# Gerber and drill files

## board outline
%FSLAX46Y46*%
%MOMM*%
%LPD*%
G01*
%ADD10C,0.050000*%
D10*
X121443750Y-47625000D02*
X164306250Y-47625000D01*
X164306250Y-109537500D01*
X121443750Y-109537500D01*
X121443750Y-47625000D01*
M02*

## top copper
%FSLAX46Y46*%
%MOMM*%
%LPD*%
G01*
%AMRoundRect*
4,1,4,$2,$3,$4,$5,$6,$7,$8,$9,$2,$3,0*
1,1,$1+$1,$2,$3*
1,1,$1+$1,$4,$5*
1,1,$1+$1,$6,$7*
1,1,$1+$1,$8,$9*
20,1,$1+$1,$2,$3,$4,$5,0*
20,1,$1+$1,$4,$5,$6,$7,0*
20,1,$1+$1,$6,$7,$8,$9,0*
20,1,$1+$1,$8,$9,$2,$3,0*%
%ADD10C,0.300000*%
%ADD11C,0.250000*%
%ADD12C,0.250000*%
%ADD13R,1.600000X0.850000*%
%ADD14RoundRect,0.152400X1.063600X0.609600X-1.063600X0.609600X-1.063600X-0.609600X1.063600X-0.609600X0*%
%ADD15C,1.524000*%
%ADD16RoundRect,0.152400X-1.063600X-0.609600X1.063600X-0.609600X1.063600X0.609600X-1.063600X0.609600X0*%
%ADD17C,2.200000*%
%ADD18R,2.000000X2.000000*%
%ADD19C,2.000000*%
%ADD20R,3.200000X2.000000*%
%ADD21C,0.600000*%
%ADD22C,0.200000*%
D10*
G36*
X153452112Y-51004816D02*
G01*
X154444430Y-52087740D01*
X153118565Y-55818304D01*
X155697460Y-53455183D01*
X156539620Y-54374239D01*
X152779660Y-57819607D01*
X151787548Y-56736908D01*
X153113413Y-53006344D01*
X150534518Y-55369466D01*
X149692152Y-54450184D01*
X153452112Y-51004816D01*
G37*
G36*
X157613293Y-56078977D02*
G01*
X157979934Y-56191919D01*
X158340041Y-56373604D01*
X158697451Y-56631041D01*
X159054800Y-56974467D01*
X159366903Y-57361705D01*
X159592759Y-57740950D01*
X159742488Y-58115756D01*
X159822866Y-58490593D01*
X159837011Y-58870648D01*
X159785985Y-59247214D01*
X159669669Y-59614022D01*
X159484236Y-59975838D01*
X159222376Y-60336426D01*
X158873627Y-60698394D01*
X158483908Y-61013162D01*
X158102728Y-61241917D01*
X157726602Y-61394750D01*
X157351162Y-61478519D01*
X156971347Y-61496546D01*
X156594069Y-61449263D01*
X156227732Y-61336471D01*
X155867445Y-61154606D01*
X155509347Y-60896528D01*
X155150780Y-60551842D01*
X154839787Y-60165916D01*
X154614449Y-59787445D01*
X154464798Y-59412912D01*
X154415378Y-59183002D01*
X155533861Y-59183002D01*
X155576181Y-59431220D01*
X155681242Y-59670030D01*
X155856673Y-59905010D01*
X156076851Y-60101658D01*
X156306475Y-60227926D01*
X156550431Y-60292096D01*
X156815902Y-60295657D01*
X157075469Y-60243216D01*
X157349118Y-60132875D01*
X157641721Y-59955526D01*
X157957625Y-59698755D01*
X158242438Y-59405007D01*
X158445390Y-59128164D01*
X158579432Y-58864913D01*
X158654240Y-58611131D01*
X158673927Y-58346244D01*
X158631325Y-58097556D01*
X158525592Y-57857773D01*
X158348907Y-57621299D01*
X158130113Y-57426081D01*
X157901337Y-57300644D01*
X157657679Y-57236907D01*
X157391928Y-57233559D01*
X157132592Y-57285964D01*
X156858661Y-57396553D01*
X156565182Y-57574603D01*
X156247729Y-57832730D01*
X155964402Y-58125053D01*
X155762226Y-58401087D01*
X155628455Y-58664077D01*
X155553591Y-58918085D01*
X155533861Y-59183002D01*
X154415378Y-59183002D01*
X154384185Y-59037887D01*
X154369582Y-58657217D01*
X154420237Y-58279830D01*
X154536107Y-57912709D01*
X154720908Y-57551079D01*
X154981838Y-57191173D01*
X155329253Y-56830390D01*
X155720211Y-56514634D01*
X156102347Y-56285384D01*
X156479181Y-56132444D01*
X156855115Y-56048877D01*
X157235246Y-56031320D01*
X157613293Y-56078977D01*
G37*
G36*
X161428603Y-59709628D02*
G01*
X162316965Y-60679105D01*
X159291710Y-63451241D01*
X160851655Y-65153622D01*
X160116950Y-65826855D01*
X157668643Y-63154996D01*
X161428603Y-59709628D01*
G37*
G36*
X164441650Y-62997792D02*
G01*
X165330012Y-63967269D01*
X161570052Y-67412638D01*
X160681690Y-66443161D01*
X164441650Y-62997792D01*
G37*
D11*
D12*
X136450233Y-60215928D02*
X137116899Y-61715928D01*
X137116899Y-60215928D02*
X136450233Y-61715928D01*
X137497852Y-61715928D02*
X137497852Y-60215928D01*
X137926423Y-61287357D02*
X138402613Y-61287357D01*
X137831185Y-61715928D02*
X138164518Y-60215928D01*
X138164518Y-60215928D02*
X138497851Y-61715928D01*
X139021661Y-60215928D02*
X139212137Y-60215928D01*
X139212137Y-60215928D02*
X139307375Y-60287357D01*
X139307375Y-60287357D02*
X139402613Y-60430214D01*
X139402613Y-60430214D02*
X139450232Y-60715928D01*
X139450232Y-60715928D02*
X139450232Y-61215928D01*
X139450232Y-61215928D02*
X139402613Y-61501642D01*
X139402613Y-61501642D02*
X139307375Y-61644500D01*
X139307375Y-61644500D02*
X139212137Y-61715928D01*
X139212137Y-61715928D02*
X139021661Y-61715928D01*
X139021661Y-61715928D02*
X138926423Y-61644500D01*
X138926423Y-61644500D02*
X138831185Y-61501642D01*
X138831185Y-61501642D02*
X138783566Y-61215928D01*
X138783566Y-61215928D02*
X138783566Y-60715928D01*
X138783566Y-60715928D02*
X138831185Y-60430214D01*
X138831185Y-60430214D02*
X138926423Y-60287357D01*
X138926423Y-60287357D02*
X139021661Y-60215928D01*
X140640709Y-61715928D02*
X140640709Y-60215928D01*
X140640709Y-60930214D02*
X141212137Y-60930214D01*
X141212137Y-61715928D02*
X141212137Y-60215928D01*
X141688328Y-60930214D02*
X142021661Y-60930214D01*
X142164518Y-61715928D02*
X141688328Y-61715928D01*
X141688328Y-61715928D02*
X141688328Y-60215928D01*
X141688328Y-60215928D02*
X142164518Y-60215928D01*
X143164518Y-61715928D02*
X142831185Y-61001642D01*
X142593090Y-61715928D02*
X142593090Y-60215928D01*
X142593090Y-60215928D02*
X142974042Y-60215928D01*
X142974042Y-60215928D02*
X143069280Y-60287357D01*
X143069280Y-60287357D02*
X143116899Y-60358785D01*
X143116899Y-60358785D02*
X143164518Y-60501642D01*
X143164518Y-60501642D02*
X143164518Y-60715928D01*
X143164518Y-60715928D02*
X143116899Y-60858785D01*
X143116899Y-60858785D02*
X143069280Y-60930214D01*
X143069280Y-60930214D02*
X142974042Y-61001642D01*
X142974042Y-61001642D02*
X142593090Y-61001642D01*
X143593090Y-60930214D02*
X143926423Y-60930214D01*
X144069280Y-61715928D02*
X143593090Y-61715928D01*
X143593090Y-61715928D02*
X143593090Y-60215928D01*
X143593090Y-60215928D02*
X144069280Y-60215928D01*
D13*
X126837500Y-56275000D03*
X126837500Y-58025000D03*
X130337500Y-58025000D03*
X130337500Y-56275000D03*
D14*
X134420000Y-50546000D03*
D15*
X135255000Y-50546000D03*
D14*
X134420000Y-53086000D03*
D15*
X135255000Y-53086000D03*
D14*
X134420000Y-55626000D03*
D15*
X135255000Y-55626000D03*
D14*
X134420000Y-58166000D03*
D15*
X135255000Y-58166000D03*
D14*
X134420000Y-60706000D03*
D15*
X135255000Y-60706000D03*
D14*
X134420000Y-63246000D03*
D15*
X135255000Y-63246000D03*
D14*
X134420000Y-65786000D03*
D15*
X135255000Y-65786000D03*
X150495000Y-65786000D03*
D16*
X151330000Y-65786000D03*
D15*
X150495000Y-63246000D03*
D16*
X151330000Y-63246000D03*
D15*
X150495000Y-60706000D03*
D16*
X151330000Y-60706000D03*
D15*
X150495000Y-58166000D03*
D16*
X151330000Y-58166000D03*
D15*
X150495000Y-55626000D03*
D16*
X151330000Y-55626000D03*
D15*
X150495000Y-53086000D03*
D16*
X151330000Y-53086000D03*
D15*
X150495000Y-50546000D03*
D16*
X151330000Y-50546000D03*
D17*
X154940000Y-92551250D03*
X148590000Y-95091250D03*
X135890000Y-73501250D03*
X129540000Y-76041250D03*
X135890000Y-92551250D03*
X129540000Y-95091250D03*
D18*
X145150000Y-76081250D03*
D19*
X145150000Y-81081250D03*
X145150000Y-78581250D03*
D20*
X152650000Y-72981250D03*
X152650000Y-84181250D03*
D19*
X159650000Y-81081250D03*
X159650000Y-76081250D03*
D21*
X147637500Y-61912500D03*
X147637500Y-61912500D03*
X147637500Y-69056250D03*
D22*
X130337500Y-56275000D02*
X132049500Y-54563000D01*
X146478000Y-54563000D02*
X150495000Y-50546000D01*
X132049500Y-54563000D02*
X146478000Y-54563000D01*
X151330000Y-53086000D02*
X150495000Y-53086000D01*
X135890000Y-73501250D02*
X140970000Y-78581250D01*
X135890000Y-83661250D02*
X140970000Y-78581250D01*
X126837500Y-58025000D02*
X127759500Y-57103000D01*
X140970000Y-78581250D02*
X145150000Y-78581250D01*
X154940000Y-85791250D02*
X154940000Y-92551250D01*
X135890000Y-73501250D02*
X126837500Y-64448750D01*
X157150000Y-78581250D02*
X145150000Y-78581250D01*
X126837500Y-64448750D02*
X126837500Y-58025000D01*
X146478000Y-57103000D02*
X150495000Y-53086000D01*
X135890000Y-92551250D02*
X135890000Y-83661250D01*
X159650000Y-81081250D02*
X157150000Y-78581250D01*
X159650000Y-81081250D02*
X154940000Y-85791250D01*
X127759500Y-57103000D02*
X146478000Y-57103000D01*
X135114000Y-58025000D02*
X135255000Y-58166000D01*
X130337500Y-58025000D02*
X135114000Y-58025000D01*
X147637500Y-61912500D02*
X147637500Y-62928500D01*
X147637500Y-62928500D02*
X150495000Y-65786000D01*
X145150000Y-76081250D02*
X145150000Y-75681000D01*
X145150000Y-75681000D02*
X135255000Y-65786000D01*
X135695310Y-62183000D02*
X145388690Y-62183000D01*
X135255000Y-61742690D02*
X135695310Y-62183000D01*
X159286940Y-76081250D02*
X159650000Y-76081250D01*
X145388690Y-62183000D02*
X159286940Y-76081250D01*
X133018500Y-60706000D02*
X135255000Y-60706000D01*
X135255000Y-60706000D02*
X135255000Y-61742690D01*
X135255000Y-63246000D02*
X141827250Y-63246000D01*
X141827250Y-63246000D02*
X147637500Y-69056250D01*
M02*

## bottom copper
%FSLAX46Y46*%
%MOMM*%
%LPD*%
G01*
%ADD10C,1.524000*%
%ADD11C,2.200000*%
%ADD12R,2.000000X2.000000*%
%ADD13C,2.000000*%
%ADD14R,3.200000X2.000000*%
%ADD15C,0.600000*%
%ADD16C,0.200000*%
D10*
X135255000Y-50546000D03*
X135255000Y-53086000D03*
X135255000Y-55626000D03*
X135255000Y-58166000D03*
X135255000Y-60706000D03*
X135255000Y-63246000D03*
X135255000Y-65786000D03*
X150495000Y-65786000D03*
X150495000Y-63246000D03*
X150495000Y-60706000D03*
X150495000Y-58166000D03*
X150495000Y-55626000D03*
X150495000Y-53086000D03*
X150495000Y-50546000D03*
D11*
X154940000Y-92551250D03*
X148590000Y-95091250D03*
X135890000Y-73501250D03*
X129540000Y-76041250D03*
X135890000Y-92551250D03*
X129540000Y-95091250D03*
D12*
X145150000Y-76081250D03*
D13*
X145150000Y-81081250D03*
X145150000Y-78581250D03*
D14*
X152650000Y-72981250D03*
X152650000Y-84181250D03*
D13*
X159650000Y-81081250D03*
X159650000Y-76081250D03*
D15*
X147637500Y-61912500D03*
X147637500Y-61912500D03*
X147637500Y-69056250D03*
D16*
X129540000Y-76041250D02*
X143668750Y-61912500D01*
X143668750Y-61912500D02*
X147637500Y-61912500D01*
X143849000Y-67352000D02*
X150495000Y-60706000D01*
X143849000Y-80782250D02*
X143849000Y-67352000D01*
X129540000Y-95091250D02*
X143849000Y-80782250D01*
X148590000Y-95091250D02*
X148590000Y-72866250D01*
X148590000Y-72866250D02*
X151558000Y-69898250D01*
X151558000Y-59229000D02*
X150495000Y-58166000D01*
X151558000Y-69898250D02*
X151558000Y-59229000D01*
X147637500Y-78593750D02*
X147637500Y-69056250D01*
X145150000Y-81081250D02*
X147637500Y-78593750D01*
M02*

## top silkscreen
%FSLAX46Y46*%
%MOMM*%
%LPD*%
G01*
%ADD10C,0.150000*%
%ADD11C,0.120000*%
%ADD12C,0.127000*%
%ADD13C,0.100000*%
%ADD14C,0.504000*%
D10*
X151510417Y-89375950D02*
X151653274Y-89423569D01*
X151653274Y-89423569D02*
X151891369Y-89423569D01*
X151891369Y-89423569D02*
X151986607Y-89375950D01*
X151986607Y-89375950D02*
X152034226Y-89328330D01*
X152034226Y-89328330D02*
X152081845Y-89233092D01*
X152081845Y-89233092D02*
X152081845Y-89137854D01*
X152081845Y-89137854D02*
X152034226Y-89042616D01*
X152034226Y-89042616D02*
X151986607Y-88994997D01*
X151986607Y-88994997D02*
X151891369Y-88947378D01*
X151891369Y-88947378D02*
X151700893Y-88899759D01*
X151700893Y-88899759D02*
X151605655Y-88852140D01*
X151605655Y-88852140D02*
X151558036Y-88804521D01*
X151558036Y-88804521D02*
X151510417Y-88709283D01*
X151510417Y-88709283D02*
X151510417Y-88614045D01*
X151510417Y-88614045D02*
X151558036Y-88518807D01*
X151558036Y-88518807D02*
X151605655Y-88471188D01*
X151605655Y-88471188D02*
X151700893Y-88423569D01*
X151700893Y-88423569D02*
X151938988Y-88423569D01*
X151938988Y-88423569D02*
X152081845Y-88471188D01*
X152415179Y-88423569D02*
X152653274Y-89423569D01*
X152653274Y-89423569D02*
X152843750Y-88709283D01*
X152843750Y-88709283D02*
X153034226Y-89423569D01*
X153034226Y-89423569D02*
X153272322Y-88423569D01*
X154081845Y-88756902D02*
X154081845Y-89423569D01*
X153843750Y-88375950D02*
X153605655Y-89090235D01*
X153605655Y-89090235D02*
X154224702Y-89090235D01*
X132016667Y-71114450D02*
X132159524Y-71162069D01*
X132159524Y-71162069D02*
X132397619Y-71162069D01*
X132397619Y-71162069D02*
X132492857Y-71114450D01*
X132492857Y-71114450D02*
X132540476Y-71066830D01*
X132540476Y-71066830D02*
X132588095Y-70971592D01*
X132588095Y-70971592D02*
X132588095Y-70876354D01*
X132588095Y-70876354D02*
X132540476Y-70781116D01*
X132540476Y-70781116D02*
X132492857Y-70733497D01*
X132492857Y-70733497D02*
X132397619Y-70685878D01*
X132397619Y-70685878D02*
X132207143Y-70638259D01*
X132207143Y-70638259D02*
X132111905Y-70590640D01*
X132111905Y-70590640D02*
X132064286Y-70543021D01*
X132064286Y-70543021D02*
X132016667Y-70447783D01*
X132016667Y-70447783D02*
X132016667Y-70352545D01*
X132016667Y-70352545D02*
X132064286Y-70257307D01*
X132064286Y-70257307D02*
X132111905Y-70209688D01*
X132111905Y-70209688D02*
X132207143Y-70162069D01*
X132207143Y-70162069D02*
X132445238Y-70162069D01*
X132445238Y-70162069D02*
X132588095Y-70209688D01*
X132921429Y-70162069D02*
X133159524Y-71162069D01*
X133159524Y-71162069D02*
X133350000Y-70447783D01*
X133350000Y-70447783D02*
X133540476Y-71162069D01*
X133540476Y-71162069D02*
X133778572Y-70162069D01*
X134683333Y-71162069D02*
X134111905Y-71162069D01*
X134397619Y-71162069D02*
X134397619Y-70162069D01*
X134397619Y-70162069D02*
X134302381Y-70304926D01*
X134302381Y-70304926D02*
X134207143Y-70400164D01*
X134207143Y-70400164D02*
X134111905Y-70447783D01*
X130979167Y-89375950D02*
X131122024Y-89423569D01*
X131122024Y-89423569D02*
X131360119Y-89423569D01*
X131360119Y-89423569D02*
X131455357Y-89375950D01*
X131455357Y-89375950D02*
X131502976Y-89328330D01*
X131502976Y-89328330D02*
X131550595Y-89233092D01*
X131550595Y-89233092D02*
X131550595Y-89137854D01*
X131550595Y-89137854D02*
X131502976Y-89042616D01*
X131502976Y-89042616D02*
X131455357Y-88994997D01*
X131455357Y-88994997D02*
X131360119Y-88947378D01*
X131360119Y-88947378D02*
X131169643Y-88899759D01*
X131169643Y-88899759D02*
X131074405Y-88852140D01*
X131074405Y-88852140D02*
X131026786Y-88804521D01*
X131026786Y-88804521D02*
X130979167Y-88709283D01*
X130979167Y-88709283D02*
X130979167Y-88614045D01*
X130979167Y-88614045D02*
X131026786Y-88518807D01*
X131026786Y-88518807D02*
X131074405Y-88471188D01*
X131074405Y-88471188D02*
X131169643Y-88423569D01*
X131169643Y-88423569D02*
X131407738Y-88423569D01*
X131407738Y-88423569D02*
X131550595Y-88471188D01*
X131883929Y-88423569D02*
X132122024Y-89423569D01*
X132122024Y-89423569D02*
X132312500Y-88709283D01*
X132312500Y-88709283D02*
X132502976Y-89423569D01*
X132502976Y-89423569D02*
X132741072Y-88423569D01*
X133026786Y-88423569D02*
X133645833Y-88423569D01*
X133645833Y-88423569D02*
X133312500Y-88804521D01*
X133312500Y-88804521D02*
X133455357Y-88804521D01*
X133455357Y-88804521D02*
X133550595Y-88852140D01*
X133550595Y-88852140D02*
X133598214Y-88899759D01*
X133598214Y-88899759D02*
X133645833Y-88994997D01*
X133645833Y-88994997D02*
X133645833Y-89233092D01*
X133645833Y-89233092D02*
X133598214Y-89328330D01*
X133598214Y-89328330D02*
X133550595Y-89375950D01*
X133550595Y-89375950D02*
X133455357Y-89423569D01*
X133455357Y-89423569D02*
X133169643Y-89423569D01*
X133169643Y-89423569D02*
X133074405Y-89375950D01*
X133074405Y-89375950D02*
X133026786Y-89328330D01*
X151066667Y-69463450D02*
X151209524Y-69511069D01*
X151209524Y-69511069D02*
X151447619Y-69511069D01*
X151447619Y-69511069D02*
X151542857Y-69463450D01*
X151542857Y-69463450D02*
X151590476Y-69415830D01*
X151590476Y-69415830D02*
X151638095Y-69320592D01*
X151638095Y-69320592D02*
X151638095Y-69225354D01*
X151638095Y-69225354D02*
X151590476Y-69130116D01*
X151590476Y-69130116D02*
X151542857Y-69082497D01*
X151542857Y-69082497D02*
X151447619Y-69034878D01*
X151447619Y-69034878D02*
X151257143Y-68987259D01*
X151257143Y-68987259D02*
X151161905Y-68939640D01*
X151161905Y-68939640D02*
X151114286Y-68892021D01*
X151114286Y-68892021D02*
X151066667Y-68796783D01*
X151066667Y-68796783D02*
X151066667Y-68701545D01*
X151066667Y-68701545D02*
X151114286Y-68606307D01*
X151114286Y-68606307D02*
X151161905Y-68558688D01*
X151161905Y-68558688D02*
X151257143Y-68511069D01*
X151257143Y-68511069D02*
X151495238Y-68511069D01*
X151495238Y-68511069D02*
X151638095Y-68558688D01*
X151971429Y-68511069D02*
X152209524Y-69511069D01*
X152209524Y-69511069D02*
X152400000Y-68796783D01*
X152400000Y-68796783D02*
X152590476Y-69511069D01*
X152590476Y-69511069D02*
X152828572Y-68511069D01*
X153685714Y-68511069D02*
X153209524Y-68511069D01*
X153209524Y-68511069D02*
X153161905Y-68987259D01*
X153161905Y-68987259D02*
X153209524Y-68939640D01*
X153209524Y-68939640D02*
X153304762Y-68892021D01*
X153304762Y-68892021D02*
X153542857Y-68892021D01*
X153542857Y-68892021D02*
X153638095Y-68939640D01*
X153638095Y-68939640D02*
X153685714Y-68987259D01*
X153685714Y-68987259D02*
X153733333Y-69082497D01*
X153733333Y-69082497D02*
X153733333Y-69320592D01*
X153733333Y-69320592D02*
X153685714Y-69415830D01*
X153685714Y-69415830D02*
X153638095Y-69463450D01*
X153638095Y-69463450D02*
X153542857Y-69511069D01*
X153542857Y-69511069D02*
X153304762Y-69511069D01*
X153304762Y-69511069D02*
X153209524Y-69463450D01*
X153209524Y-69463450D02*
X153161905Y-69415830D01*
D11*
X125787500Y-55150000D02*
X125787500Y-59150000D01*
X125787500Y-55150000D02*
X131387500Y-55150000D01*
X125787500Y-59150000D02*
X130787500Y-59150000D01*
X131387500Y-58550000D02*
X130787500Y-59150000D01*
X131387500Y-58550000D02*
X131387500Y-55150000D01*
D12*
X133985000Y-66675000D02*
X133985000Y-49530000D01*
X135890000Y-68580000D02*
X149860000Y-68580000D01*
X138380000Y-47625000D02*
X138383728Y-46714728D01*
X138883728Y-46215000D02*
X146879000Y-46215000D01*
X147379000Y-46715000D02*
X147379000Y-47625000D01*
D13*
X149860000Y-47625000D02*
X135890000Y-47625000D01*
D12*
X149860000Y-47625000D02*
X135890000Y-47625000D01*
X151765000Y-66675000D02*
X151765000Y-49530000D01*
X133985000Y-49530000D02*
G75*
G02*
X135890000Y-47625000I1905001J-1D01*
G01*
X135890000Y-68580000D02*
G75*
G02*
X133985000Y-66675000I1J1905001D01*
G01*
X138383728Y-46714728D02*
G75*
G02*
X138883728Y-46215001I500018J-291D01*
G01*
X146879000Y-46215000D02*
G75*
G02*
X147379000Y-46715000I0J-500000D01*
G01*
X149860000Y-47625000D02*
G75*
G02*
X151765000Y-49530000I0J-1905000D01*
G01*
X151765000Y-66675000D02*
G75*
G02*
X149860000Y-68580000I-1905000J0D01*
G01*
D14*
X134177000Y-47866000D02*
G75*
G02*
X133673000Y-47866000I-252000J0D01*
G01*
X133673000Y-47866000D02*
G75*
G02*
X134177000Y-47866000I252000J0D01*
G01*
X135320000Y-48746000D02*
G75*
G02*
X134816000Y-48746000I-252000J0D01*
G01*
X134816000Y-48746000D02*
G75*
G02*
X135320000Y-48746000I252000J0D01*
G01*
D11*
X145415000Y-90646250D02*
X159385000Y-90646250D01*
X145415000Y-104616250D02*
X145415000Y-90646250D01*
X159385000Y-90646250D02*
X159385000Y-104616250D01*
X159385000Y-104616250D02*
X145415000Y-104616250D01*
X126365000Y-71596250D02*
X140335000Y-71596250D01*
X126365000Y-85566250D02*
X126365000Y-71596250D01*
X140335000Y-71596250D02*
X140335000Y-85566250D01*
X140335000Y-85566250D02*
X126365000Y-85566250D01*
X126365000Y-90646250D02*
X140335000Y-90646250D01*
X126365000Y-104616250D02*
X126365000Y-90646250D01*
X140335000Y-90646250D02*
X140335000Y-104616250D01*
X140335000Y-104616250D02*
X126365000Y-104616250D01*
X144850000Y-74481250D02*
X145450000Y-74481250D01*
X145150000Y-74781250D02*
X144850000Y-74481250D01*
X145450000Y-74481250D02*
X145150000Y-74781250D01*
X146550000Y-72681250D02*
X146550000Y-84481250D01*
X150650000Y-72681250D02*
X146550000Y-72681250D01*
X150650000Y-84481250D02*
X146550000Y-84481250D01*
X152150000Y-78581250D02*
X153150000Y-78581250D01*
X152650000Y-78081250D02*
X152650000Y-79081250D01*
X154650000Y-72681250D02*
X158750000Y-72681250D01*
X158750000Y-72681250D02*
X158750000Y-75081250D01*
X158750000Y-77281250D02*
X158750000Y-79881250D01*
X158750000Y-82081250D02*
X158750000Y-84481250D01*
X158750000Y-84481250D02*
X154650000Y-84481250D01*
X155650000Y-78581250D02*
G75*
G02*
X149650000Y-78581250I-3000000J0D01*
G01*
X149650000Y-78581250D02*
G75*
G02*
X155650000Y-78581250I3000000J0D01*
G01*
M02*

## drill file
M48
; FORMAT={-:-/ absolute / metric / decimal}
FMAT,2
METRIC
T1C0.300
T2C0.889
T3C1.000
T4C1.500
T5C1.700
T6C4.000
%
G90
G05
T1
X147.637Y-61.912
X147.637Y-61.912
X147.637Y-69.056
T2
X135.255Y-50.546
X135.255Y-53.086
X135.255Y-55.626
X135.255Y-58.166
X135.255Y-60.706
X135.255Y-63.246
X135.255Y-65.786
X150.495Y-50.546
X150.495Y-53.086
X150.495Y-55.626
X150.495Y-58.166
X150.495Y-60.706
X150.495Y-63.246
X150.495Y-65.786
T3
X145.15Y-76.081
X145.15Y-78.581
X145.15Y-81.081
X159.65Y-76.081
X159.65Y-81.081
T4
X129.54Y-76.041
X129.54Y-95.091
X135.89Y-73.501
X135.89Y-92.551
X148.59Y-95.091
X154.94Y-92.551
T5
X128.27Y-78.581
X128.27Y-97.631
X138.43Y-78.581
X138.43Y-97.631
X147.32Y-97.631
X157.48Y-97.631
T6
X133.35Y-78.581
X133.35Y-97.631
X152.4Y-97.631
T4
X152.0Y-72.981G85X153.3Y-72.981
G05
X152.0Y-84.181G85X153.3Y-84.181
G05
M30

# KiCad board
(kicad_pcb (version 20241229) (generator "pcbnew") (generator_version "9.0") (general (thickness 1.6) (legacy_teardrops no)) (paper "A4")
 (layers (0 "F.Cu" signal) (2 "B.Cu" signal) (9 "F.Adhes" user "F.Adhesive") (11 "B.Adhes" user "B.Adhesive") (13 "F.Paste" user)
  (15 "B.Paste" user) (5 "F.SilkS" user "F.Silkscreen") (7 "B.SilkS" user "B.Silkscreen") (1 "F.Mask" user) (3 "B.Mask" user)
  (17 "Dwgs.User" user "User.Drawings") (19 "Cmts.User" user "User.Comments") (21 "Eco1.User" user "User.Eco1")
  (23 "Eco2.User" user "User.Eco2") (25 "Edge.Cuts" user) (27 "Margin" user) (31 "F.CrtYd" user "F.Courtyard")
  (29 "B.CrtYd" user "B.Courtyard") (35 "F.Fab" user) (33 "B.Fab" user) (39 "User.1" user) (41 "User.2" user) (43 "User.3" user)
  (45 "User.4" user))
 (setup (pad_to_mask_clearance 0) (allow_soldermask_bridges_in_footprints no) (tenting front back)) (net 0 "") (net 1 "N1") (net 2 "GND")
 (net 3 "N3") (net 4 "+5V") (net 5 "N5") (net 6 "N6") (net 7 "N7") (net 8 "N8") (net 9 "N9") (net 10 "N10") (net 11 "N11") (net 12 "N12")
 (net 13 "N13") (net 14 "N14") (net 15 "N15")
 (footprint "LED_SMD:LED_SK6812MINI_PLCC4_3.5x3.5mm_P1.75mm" (layer "F.Cu") (at 128.5875 57.15)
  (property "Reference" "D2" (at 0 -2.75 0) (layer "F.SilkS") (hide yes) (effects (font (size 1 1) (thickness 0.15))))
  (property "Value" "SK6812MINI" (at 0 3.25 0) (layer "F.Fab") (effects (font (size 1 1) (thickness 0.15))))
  (fp_line (start -2.8 -2) (end -2.8 2) (stroke (width 0.12) (type default)) (layer "F.SilkS"))
  (fp_line (start -2.8 -2) (end 2.8 -2) (stroke (width 0.12) (type solid)) (layer "F.SilkS"))
  (fp_line (start -2.8 2) (end 2.2 2) (stroke (width 0.12) (type solid)) (layer "F.SilkS"))
  (fp_line (start 2.8 1.4) (end 2.2 2) (stroke (width 0.12) (type default)) (layer "F.SilkS"))
  (fp_line (start 2.8 1.4) (end 2.8 -2) (stroke (width 0.12) (type solid)) (layer "F.SilkS"))
  (pad "1" smd rect (at -1.75 -0.875) (size 1.6 0.85) (layers "F.Cu" "F.Mask" "F.Paste") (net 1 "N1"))
  (pad "2" smd rect (at -1.75 0.875) (size 1.6 0.85) (layers "F.Cu" "F.Mask" "F.Paste") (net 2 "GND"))
  (pad "3" smd rect (at 1.75 0.875) (size 1.6 0.85) (layers "F.Cu" "F.Mask" "F.Paste") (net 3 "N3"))
  (pad "4" smd rect (at 1.75 -0.875) (size 1.6 0.85) (layers "F.Cu" "F.Mask" "F.Paste") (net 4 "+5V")))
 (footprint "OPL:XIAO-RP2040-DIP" (layer "F.Cu") (at 142.875 58.166)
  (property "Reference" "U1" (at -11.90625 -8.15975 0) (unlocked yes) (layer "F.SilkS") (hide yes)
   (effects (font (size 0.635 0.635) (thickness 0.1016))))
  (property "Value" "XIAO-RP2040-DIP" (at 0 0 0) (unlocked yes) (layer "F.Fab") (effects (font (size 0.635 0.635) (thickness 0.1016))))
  (fp_line (start -8.89 8.509) (end -8.89 -8.636) (stroke (width 0.127) (type solid)) (layer "F.SilkS"))
  (fp_line (start -6.985 10.414) (end 6.985 10.414) (stroke (width 0.127) (type solid)) (layer "F.SilkS"))
  (fp_line (start -4.495 -10.541) (end -4.491272 -11.451272) (stroke (width 0.127) (type solid)) (layer "F.SilkS"))
  (fp_line (start -3.991272 -11.951) (end 4.004 -11.951) (stroke (width 0.127) (type solid)) (layer "F.SilkS"))
  (fp_line (start 4.504 -11.451) (end 4.504 -10.541) (stroke (width 0.127) (type solid)) (layer "F.SilkS"))
  (fp_line (start 6.985 -10.541) (end -6.985 -10.541) (stroke (width 0.1) (type solid)) (layer "F.SilkS"))
  (fp_line (start 6.985 -10.541) (end -6.985 -10.541) (stroke (width 0.127) (type solid)) (layer "F.SilkS"))
  (fp_line (start 8.89 8.509) (end 8.89 -8.636) (stroke (width 0.127) (type solid)) (layer "F.SilkS"))
  (fp_arc (start -8.89 -8.636) (mid -8.332038 -9.983038) (end -6.985 -10.541) (stroke (width 0.127) (type solid)) (layer "F.SilkS"))
  (fp_arc (start -6.985 10.414) (mid -8.332038 9.856038) (end -8.89 8.509) (stroke (width 0.127) (type solid)) (layer "F.SilkS"))
  (fp_arc (start -4.491272 -11.451272) (mid -4.344728 -11.80464) (end -3.991272 -11.951) (stroke (width 0.127) (type default))
   (layer "F.SilkS"))
  (fp_arc (start 4.004 -11.951) (mid 4.357553 -11.804553) (end 4.504 -11.451) (stroke (width 0.127) (type default)) (layer "F.SilkS"))
  (fp_arc (start 6.985 -10.541) (mid 8.332038 -9.983038) (end 8.89 -8.636) (stroke (width 0.127) (type solid)) (layer "F.SilkS"))
  (fp_arc (start 8.89 8.509) (mid 8.332038 9.856038) (end 6.985 10.414) (stroke (width 0.127) (type solid)) (layer "F.SilkS"))
  (fp_circle (center -8.95 -10.3) (end -8.95 -10.554) (stroke (width 0.5) (type solid)) (fill yes) (layer "F.SilkS"))
  (fp_circle (center -7.807 -9.42) (end -7.807 -9.674) (stroke (width 0.5) (type solid)) (fill yes) (layer "F.SilkS"))
  (pad "1" smd roundrect (at -8.455 -7.62 180) (size 2.432 1.524) (layers "F.Cu" "F.Mask") (roundrect_rratio 0.1) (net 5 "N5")
   (thermal_bridge_angle 45))
  (pad "1" thru_hole circle (at -7.62 -7.62 180) (size 1.524 1.524) (drill 0.889) (layers "*.Cu" "*.Mask") (remove_unused_layers no)
   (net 5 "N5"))
  (pad "2" smd roundrect (at -8.455 -5.08 180) (size 2.432 1.524) (layers "F.Cu" "F.Mask") (roundrect_rratio 0.1) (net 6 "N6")
   (thermal_bridge_angle 45))
  (pad "2" thru_hole circle (at -7.62 -5.08 180) (size 1.524 1.524) (drill 0.889) (layers "*.Cu" "*.Mask") (remove_unused_layers no)
   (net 6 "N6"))
  (pad "3" smd roundrect (at -8.455 -2.54 180) (size 2.432 1.524) (layers "F.Cu" "F.Mask") (roundrect_rratio 0.1) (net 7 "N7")
   (thermal_bridge_angle 45))
  (pad "3" thru_hole circle (at -7.62 -2.54 180) (size 1.524 1.524) (drill 0.889) (layers "*.Cu" "*.Mask") (remove_unused_layers no)
   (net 7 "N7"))
  (pad "4" smd roundrect (at -8.455 0 180) (size 2.432 1.524) (layers "F.Cu" "F.Mask") (roundrect_rratio 0.1) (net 3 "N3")
   (thermal_bridge_angle 45))
  (pad "4" thru_hole circle (at -7.62 0 180) (size 1.524 1.524) (drill 0.889) (layers "*.Cu" "*.Mask") (remove_unused_layers no)
   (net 3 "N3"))
  (pad "5" smd roundrect (at -8.455 2.54 180) (size 2.432 1.524) (layers "F.Cu" "F.Mask") (roundrect_rratio 0.1) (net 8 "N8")
   (thermal_bridge_angle 45))
  (pad "5" thru_hole circle (at -7.62 2.54 180) (size 1.524 1.524) (drill 0.889) (layers "*.Cu" "*.Mask") (remove_unused_layers no)
   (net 8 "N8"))
  (pad "6" smd roundrect (at -8.455 5.08 180) (size 2.432 1.524) (layers "F.Cu" "F.Mask") (roundrect_rratio 0.1) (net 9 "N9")
   (thermal_bridge_angle 45))
  (pad "6" thru_hole circle (at -7.62 5.08 180) (size 1.524 1.524) (drill 0.889) (layers "*.Cu" "*.Mask") (remove_unused_layers no)
   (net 9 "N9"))
  (pad "7" smd roundrect (at -8.455 7.62 180) (size 2.432 1.524) (layers "F.Cu" "F.Mask") (roundrect_rratio 0.1) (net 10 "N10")
   (thermal_bridge_angle 45))
  (pad "7" thru_hole circle (at -7.62 7.62 180) (size 1.524 1.524) (drill 0.889) (layers "*.Cu" "*.Mask") (remove_unused_layers no)
   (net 10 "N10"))
  (pad "8" thru_hole circle (at 7.62 7.62) (size 1.524 1.524) (drill 0.889) (layers "*.Cu" "*.Mask") (remove_unused_layers no)
   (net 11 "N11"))
  (pad "8" smd roundrect (at 8.455 7.62) (size 2.432 1.524) (layers "F.Cu" "F.Mask") (roundrect_rratio 0.1) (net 11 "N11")
   (thermal_bridge_angle 45))
  (pad "9" thru_hole circle (at 7.62 5.08) (size 1.524 1.524) (drill 0.889) (layers "*.Cu" "*.Mask") (remove_unused_layers no)
   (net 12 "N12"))
  (pad "9" smd roundrect (at 8.455 5.08) (size 2.432 1.524) (layers "F.Cu" "F.Mask") (roundrect_rratio 0.1) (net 12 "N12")
   (thermal_bridge_angle 45))
  (pad "10" thru_hole circle (at 7.62 2.54) (size 1.524 1.524) (drill 0.889) (layers "*.Cu" "*.Mask") (remove_unused_layers no)
   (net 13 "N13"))
  (pad "10" smd roundrect (at 8.455 2.54) (size 2.432 1.524) (layers "F.Cu" "F.Mask") (roundrect_rratio 0.1) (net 13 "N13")
   (thermal_bridge_angle 45))
  (pad "11" thru_hole circle (at 7.62 0) (size 1.524 1.524) (drill 0.889) (layers "*.Cu" "*.Mask") (remove_unused_layers no) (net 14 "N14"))
  (pad "11" smd roundrect (at 8.455 0) (size 2.432 1.524) (layers "F.Cu" "F.Mask") (roundrect_rratio 0.1) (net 14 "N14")
   (thermal_bridge_angle 45))
  (pad "12" thru_hole circle (at 7.62 -2.54) (size 1.524 1.524) (drill 0.889) (layers "*.Cu" "*.Mask") (remove_unused_layers no)
   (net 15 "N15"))
  (pad "12" smd roundrect (at 8.455 -2.54) (size 2.432 1.524) (layers "F.Cu" "F.Mask") (roundrect_rratio 0.1) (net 15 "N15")
   (thermal_bridge_angle 45))
  (pad "13" thru_hole circle (at 7.62 -5.08) (size 1.524 1.524) (drill 0.889) (layers "*.Cu" "*.Mask") (remove_unused_layers no)
   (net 2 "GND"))
  (pad "13" smd roundrect (at 8.455 -5.08) (size 2.432 1.524) (layers "F.Cu" "F.Mask") (roundrect_rratio 0.1) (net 2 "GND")
   (thermal_bridge_angle 45))
  (pad "14" thru_hole circle (at 7.62 -7.62) (size 1.524 1.524) (drill 0.889) (layers "*.Cu" "*.Mask") (remove_unused_layers no)
   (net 4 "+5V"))
  (pad "14" smd roundrect (at 8.455 -7.62) (size 2.432 1.524) (layers "F.Cu" "F.Mask") (roundrect_rratio 0.1) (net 4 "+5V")
   (thermal_bridge_angle 45)))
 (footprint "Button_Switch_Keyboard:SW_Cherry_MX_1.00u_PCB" (layer "F.Cu") (at 154.94 92.55125)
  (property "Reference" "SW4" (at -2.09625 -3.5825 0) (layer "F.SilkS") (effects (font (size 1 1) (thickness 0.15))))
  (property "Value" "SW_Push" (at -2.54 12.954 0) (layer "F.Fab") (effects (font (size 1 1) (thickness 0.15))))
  (fp_line (start -9.525 -1.905) (end 4.445 -1.905) (stroke (width 0.12) (type solid)) (layer "F.SilkS"))
  (fp_line (start -9.525 12.065) (end -9.525 -1.905) (stroke (width 0.12) (type solid)) (layer "F.SilkS"))
  (fp_line (start 4.445 -1.905) (end 4.445 12.065) (stroke (width 0.12) (type solid)) (layer "F.SilkS"))
  (fp_line (start 4.445 12.065) (end -9.525 12.065) (stroke (width 0.12) (type solid)) (layer "F.SilkS"))
  (pad "" np_thru_hole circle (at -7.62 5.08) (size 1.7 1.7) (drill 1.7) (layers "*.Cu" "*.Mask"))
  (pad "" np_thru_hole circle (at -2.54 5.08) (size 4 4) (drill 4) (layers "*.Cu" "*.Mask"))
  (pad "" np_thru_hole circle (at 2.54 5.08) (size 1.7 1.7) (drill 1.7) (layers "*.Cu" "*.Mask"))
  (pad "1" thru_hole circle (at 0 0) (size 2.2 2.2) (drill 1.5) (layers "*.Cu" "*.Mask") (remove_unused_layers no) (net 2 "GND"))
  (pad "2" thru_hole circle (at -6.35 2.54) (size 2.2 2.2) (drill 1.5) (layers "*.Cu" "*.Mask") (remove_unused_layers no) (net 14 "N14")))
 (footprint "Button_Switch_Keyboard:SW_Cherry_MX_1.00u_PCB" (layer "F.Cu") (at 135.89 73.50125)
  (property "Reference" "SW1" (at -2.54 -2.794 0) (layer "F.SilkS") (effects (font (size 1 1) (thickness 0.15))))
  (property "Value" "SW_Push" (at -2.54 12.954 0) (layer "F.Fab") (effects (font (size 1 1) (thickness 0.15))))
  (fp_line (start -9.525 -1.905) (end 4.445 -1.905) (stroke (width 0.12) (type solid)) (layer "F.SilkS"))
  (fp_line (start -9.525 12.065) (end -9.525 -1.905) (stroke (width 0.12) (type solid)) (layer "F.SilkS"))
  (fp_line (start 4.445 -1.905) (end 4.445 12.065) (stroke (width 0.12) (type solid)) (layer "F.SilkS"))
  (fp_line (start 4.445 12.065) (end -9.525 12.065) (stroke (width 0.12) (type solid)) (layer "F.SilkS"))
  (pad "" np_thru_hole circle (at -7.62 5.08) (size 1.7 1.7) (drill 1.7) (layers "*.Cu" "*.Mask"))
  (pad "" np_thru_hole circle (at -2.54 5.08) (size 4 4) (drill 4) (layers "*.Cu" "*.Mask"))
  (pad "" np_thru_hole circle (at 2.54 5.08) (size 1.7 1.7) (drill 1.7) (layers "*.Cu" "*.Mask"))
  (pad "1" thru_hole circle (at 0 0) (size 2.2 2.2) (drill 1.5) (layers "*.Cu" "*.Mask") (remove_unused_layers no) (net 2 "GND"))
  (pad "2" thru_hole circle (at -6.35 2.54) (size 2.2 2.2) (drill 1.5) (layers "*.Cu" "*.Mask") (remove_unused_layers no) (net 11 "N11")))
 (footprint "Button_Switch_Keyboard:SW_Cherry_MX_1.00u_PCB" (layer "F.Cu") (at 135.89 92.55125)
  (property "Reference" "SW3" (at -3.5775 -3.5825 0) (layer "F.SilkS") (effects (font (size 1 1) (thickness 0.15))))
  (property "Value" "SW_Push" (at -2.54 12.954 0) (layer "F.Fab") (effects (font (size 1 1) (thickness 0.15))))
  (fp_line (start -9.525 -1.905) (end 4.445 -1.905) (stroke (width 0.12) (type solid)) (layer "F.SilkS"))
  (fp_line (start -9.525 12.065) (end -9.525 -1.905) (stroke (width 0.12) (type solid)) (layer "F.SilkS"))
  (fp_line (start 4.445 -1.905) (end 4.445 12.065) (stroke (width 0.12) (type solid)) (layer "F.SilkS"))
  (fp_line (start 4.445 12.065) (end -9.525 12.065) (stroke (width 0.12) (type solid)) (layer "F.SilkS"))
  (pad "" np_thru_hole circle (at -7.62 5.08) (size 1.7 1.7) (drill 1.7) (layers "*.Cu" "*.Mask"))
  (pad "" np_thru_hole circle (at -2.54 5.08) (size 4 4) (drill 4) (layers "*.Cu" "*.Mask"))
  (pad "" np_thru_hole circle (at 2.54 5.08) (size 1.7 1.7) (drill 1.7) (layers "*.Cu" "*.Mask"))
  (pad "1" thru_hole circle (at 0 0) (size 2.2 2.2) (drill 1.5) (layers "*.Cu" "*.Mask") (remove_unused_layers no) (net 2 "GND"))
  (pad "2" thru_hole circle (at -6.35 2.54) (size 2.2 2.2) (drill 1.5) (layers "*.Cu" "*.Mask") (remove_unused_layers no) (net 13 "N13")))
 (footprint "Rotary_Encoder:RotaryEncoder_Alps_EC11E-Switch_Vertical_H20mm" (layer "F.Cu") (at 145.15 76.08125)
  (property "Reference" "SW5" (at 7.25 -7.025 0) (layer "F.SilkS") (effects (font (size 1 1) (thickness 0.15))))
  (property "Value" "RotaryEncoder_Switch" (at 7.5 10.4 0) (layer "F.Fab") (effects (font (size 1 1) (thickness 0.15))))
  (fp_line (start -0.3 -1.6) (end 0.3 -1.6) (stroke (width 0.12) (type solid)) (layer "F.SilkS"))
  (fp_line (start 0 -1.3) (end -0.3 -1.6) (stroke (width 0.12) (type solid)) (layer "F.SilkS"))
  (fp_line (start 0.3 -1.6) (end 0 -1.3) (stroke (width 0.12) (type solid)) (layer "F.SilkS"))
  (fp_line (start 1.4 -3.4) (end 1.4 8.4) (stroke (width 0.12) (type solid)) (layer "F.SilkS"))
  (fp_line (start 5.5 -3.4) (end 1.4 -3.4) (stroke (width 0.12) (type solid)) (layer "F.SilkS"))
  (fp_line (start 5.5 8.4) (end 1.4 8.4) (stroke (width 0.12) (type solid)) (layer "F.SilkS"))
  (fp_line (start 7 2.5) (end 8 2.5) (stroke (width 0.12) (type solid)) (layer "F.SilkS"))
  (fp_line (start 7.5 2) (end 7.5 3) (stroke (width 0.12) (type solid)) (layer "F.SilkS"))
  (fp_line (start 9.5 -3.4) (end 13.6 -3.4) (stroke (width 0.12) (type solid)) (layer "F.SilkS"))
  (fp_line (start 13.6 -3.4) (end 13.6 -1) (stroke (width 0.12) (type solid)) (layer "F.SilkS"))
  (fp_line (start 13.6 1.2) (end 13.6 3.8) (stroke (width 0.12) (type solid)) (layer "F.SilkS"))
  (fp_line (start 13.6 6) (end 13.6 8.4) (stroke (width 0.12) (type solid)) (layer "F.SilkS"))
  (fp_line (start 13.6 8.4) (end 9.5 8.4) (stroke (width 0.12) (type solid)) (layer "F.SilkS"))
  (fp_circle (center 7.5 2.5) (end 10.5 2.5) (stroke (width 0.12) (type solid)) (fill no) (layer "F.SilkS"))
  (pad "A" thru_hole rect (at 0 0) (size 2 2) (drill 1) (layers "*.Cu" "*.Mask") (remove_unused_layers no) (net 10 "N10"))
  (pad "B" thru_hole circle (at 0 5) (size 2 2) (drill 1) (layers "*.Cu" "*.Mask") (remove_unused_layers no) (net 9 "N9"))
  (pad "C" thru_hole circle (at 0 2.5) (size 2 2) (drill 1) (layers "*.Cu" "*.Mask") (remove_unused_layers no) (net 2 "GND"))
  (pad "MP" thru_hole rect (at 7.5 -3.1) (size 3.2 2) (drill oval 2.8 1.5) (layers "*.Cu" "*.Mask") (remove_unused_layers no))
  (pad "MP" thru_hole rect (at 7.5 8.1) (size 3.2 2) (drill oval 2.8 1.5) (layers "*.Cu" "*.Mask") (remove_unused_layers no))
  (pad "S1" thru_hole circle (at 14.5 5) (size 2 2) (drill 1) (layers "*.Cu" "*.Mask") (remove_unused_layers no) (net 2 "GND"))
  (pad "S2" thru_hole circle (at 14.5 0) (size 2 2) (drill 1) (layers "*.Cu" "*.Mask") (remove_unused_layers no) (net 8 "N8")))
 (gr_rect (start 121.44375 47.625) (end 164.30625 109.5375) (stroke (width 0.05) (type default)) (fill no) (layer "Edge.Cuts"))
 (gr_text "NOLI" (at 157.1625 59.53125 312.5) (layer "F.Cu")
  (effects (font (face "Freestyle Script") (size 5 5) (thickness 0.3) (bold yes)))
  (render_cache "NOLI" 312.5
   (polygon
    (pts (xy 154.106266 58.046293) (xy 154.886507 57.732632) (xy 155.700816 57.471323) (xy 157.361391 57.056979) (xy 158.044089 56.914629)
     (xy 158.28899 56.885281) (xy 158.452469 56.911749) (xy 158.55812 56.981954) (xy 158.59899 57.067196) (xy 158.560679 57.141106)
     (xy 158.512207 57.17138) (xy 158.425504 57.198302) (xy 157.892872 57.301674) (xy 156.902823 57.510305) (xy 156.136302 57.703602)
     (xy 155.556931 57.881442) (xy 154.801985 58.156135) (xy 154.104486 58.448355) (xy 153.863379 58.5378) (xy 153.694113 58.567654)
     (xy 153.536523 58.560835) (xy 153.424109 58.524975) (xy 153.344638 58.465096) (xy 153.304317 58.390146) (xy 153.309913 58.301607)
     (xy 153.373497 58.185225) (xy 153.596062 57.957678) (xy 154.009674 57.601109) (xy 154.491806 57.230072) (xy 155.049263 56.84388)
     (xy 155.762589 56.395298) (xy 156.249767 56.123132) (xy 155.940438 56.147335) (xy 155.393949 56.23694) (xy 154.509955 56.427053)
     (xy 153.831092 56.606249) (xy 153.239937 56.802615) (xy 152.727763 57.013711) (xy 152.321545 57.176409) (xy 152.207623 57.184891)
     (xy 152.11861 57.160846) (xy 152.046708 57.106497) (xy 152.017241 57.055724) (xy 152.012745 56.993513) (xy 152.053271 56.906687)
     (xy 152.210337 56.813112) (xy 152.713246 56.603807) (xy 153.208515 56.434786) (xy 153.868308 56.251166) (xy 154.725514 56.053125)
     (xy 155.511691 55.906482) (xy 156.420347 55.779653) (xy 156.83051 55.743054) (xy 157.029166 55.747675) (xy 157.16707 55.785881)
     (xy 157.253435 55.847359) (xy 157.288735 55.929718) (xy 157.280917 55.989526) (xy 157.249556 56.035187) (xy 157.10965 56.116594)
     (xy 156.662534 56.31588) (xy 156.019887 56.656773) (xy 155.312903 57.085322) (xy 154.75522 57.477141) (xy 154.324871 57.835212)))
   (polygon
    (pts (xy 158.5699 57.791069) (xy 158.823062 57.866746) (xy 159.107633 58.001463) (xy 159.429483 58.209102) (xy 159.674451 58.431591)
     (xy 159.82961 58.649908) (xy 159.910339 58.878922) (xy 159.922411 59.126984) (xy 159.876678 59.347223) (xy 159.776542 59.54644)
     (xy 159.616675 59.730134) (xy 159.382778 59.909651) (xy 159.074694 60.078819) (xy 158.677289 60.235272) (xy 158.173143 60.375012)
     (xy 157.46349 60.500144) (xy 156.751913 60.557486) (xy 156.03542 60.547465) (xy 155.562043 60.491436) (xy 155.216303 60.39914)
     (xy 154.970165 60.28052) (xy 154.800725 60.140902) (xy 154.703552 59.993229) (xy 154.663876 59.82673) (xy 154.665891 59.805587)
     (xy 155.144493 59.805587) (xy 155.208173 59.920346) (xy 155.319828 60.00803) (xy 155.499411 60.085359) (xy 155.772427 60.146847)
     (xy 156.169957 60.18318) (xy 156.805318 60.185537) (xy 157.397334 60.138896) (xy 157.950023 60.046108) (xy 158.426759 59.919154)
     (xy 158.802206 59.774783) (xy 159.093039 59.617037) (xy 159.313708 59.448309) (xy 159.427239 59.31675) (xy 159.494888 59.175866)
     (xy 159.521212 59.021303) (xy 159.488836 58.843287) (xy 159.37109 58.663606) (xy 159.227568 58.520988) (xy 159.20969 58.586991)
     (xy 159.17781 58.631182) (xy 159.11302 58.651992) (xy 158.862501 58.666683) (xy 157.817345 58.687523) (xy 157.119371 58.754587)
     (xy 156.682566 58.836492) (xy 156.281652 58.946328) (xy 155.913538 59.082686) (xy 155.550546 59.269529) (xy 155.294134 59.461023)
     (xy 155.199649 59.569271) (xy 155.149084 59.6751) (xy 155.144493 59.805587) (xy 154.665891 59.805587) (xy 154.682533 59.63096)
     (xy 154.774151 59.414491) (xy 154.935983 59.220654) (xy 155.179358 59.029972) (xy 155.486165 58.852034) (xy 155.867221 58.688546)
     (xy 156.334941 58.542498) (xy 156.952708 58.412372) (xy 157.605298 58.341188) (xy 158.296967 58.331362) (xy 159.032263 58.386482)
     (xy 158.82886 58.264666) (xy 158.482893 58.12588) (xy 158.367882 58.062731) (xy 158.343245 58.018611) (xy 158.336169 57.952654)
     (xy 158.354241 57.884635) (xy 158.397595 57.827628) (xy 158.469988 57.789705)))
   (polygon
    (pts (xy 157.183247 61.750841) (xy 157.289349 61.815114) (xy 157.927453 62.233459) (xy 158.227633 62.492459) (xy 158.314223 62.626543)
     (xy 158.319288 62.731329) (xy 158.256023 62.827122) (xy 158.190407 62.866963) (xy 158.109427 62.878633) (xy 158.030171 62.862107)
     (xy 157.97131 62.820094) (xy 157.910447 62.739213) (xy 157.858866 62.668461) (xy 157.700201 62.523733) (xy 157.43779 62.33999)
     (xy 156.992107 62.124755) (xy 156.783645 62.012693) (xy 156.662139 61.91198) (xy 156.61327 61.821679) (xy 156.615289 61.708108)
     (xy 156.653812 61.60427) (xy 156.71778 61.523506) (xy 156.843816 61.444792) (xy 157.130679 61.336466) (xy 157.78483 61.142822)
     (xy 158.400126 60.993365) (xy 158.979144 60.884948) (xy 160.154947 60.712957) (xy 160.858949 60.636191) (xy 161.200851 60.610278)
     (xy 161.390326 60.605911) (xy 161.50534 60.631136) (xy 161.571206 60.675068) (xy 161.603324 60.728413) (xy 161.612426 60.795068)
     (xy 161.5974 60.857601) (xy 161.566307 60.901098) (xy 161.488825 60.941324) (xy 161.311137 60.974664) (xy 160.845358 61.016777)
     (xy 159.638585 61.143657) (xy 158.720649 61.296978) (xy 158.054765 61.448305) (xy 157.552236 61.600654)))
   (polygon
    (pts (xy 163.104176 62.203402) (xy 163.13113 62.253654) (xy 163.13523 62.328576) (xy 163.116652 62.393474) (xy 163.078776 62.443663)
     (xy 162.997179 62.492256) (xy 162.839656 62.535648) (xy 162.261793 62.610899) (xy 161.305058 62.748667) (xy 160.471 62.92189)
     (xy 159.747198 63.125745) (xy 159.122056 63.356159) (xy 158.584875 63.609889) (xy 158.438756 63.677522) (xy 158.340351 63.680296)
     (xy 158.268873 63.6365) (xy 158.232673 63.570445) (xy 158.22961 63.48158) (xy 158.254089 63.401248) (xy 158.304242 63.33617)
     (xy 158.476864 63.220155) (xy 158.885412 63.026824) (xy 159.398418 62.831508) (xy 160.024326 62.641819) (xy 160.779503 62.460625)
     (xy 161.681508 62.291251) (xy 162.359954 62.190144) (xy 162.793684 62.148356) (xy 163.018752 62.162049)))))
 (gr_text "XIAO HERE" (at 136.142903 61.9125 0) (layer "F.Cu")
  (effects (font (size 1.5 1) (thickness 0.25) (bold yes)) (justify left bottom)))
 (segment (start 130.3375 56.275) (end 132.0495 54.563) (width 0.2) (layer "F.Cu") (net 4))
 (segment (start 146.478 54.563) (end 150.495 50.546) (width 0.2) (layer "F.Cu") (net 4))
 (segment (start 132.0495 54.563) (end 146.478 54.563) (width 0.2) (layer "F.Cu") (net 4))
 (segment (start 151.33 53.086) (end 150.495 53.086) (width 0.2) (layer "F.Cu") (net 2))
 (segment (start 135.89 73.50125) (end 140.97 78.58125) (width 0.2) (layer "F.Cu") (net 2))
 (segment (start 135.89 83.66125) (end 140.97 78.58125) (width 0.2) (layer "F.Cu") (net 2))
 (segment (start 126.8375 58.025) (end 127.7595 57.103) (width 0.2) (layer "F.Cu") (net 2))
 (segment (start 140.97 78.58125) (end 145.15 78.58125) (width 0.2) (layer "F.Cu") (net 2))
 (segment (start 154.94 85.79125) (end 154.94 92.55125) (width 0.2) (layer "F.Cu") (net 2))
 (segment (start 135.89 73.50125) (end 126.8375 64.44875) (width 0.2) (layer "F.Cu") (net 2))
 (segment (start 157.15 78.58125) (end 145.15 78.58125) (width 0.2) (layer "F.Cu") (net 2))
 (segment (start 126.8375 64.44875) (end 126.8375 58.025) (width 0.2) (layer "F.Cu") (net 2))
 (segment (start 146.478 57.103) (end 150.495 53.086) (width 0.2) (layer "F.Cu") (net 2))
 (segment (start 135.89 92.55125) (end 135.89 83.66125) (width 0.2) (layer "F.Cu") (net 2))
 (segment (start 159.65 81.08125) (end 157.15 78.58125) (width 0.2) (layer "F.Cu") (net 2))
 (segment (start 159.65 81.08125) (end 154.94 85.79125) (width 0.2) (layer "F.Cu") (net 2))
 (segment (start 127.7595 57.103) (end 146.478 57.103) (width 0.2) (layer "F.Cu") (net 2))
 (segment (start 135.114 58.025) (end 135.255 58.166) (width 0.2) (layer "F.Cu") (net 3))
 (segment (start 130.3375 58.025) (end 135.114 58.025) (width 0.2) (layer "F.Cu") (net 3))
 (segment (start 147.6375 61.9125) (end 147.6375 62.9285) (width 0.2) (layer "F.Cu") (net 11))
 (segment (start 147.6375 62.9285) (end 150.495 65.786) (width 0.2) (layer "F.Cu") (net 11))
 (via (at 147.6375 61.9125) (size 0.6) (drill 0.3) (layers "F.Cu" "B.Cu") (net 11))
 (via (at 147.6375 61.9125) (size 0.6) (drill 0.3) (layers "F.Cu" "B.Cu") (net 11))
 (segment (start 129.54 76.04125) (end 143.66875 61.9125) (width 0.2) (layer "B.Cu") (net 11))
 (segment (start 143.66875 61.9125) (end 147.6375 61.9125) (width 0.2) (layer "B.Cu") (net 11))
 (segment (start 143.849 67.352) (end 150.495 60.706) (width 0.2) (layer "B.Cu") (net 13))
 (segment (start 143.849 80.78225) (end 143.849 67.352) (width 0.2) (layer "B.Cu") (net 13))
 (segment (start 129.54 95.09125) (end 143.849 80.78225) (width 0.2) (layer "B.Cu") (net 13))
 (segment (start 148.59 95.09125) (end 148.59 72.86625) (width 0.2) (layer "B.Cu") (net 14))
 (segment (start 148.59 72.86625) (end 151.558 69.89825) (width 0.2) (layer "B.Cu") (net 14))
 (segment (start 151.558 59.229) (end 150.495 58.166) (width 0.2) (layer "B.Cu") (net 14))
 (segment (start 151.558 69.89825) (end 151.558 59.229) (width 0.2) (layer "B.Cu") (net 14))
 (segment (start 145.15 76.08125) (end 145.15 75.681) (width 0.2) (layer "F.Cu") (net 10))
 (segment (start 145.15 75.681) (end 135.255 65.786) (width 0.2) (layer "F.Cu") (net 10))
 (segment (start 135.69531 62.183) (end 145.38869 62.183) (width 0.2) (layer "F.Cu") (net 8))
 (segment (start 135.255 61.74269) (end 135.69531 62.183) (width 0.2) (layer "F.Cu") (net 8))
 (segment (start 159.28694 76.08125) (end 159.65 76.08125) (width 0.2) (layer "F.Cu") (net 8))
 (segment (start 145.38869 62.183) (end 159.28694 76.08125) (width 0.2) (layer "F.Cu") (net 8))
 (segment (start 133.0185 60.706) (end 135.255 60.706) (width 0.2) (layer "F.Cu") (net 8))
 (segment (start 135.255 60.706) (end 135.255 61.74269) (width 0.2) (layer "F.Cu") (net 8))
 (segment (start 135.255 63.246) (end 141.82725 63.246) (width 0.2) (layer "F.Cu") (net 9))
 (segment (start 141.82725 63.246) (end 147.6375 69.05625) (width 0.2) (layer "F.Cu") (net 9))
 (via (at 147.6375 69.05625) (size 0.6) (drill 0.3) (layers "F.Cu" "B.Cu") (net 9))
 (segment (start 147.6375 78.59375) (end 147.6375 69.05625) (width 0.2) (layer "B.Cu") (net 9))
 (segment (start 145.15 81.08125) (end 147.6375 78.59375) (width 0.2) (layer "B.Cu") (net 9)))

